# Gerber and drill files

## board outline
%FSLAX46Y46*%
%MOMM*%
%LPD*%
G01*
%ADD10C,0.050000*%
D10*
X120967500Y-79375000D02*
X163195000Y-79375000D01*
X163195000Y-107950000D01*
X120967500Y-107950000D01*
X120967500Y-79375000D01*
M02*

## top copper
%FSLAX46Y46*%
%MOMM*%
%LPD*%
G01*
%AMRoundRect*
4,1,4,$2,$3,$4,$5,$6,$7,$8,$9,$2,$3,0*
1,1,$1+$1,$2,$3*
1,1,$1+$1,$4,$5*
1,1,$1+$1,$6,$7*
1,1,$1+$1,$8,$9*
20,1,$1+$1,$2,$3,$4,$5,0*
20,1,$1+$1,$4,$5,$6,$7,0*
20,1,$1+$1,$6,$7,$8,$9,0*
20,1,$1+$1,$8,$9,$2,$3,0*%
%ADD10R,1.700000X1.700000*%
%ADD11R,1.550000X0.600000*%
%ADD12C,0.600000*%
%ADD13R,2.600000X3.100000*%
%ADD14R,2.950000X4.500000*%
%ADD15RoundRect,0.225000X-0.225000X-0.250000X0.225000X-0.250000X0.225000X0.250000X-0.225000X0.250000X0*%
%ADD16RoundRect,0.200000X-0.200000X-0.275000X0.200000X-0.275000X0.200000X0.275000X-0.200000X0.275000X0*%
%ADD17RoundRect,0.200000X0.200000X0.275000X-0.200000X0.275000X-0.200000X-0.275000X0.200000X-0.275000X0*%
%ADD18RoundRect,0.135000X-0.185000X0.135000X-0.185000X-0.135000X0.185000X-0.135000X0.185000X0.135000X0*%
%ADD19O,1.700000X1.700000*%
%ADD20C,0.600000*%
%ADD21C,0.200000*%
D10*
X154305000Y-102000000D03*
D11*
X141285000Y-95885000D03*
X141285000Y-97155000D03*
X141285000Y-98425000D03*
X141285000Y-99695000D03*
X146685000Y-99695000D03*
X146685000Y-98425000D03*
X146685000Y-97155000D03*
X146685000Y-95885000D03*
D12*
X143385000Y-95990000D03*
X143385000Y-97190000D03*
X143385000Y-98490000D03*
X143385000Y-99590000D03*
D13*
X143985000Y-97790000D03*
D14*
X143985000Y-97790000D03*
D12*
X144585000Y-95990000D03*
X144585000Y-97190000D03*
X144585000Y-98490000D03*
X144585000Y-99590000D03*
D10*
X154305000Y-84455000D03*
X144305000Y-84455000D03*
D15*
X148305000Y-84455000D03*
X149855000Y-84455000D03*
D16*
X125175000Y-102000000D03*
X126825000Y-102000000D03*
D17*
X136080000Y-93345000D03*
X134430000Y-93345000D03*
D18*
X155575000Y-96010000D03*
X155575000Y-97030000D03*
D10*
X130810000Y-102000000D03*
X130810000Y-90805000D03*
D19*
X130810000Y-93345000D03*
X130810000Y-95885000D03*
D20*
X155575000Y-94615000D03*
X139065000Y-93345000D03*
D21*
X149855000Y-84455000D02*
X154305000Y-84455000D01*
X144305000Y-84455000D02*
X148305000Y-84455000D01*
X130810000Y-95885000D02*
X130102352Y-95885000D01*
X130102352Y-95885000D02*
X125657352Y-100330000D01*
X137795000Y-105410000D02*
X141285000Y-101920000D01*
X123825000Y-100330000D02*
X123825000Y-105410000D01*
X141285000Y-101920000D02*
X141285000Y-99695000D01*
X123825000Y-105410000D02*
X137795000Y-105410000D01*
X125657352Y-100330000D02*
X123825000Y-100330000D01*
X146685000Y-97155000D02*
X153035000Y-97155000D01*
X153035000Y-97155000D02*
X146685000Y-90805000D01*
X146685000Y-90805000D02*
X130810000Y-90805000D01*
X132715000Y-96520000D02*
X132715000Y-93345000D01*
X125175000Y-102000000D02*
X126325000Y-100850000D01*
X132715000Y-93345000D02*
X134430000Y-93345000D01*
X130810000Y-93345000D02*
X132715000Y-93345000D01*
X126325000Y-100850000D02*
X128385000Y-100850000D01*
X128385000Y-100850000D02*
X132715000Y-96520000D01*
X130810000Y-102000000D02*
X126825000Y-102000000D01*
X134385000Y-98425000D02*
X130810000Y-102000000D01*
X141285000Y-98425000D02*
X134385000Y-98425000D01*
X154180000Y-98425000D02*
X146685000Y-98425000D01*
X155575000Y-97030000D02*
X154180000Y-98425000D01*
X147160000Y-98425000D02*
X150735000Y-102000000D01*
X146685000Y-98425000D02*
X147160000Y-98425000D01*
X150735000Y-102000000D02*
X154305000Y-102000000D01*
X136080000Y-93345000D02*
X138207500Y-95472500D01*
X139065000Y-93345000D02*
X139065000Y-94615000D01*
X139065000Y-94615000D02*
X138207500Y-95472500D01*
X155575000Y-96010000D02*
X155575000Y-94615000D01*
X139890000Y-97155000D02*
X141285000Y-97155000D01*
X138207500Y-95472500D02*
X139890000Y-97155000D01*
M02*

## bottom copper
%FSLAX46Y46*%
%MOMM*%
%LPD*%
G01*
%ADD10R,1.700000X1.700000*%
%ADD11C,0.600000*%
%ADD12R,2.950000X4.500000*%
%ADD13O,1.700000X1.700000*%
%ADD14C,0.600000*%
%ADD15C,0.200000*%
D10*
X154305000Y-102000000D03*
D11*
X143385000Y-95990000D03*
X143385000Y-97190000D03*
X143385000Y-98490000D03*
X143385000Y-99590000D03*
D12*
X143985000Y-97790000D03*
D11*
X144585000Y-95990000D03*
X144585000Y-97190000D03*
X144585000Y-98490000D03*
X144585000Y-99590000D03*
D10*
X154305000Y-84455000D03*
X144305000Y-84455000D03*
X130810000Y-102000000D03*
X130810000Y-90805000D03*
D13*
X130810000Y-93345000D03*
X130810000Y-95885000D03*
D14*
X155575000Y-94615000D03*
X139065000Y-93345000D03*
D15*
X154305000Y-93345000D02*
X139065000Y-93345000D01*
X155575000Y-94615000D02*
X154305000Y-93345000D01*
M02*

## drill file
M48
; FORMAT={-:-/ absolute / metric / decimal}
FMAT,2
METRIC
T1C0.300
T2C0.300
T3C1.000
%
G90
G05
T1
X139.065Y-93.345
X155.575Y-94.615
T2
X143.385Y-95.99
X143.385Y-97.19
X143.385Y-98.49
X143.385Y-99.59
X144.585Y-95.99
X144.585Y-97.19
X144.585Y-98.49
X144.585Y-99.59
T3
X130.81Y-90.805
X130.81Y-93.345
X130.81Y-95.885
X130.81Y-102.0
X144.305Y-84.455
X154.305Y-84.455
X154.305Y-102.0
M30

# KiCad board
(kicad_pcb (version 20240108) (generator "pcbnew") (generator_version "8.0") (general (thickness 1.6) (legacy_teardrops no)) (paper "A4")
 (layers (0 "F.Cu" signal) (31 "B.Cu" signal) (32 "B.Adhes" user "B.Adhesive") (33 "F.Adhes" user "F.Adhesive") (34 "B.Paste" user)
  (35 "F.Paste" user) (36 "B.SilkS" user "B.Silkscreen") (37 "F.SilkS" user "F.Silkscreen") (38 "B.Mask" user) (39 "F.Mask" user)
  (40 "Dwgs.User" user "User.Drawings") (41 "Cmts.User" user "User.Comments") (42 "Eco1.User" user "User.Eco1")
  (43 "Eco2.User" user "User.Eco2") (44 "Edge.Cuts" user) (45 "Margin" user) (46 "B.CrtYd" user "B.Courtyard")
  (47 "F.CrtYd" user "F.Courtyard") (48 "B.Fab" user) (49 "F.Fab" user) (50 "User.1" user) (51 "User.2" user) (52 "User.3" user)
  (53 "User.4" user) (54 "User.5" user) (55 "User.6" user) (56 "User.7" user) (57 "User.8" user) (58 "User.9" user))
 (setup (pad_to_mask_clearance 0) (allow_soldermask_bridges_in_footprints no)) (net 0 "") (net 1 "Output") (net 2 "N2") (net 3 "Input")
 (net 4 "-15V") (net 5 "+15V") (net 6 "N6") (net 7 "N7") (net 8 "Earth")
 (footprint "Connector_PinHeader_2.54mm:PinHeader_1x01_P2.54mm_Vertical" (layer "F.Cu") (at 154.305 102)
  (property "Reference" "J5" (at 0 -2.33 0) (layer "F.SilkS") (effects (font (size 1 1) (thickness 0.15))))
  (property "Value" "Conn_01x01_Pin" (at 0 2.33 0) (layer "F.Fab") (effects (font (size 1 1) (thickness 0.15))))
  (pad "1" thru_hole rect (at 0 0) (size 1.7 1.7) (drill 1) (layers "*.Cu" "*.Mask") (remove_unused_layers no) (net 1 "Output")))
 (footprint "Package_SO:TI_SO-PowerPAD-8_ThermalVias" (layer "F.Cu") (at 143.985 97.79)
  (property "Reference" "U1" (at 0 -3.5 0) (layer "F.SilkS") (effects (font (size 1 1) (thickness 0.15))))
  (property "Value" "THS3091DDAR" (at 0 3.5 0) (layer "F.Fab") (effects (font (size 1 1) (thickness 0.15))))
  (pad "1" smd rect (at -2.7 -1.905) (size 1.55 0.6) (layers "F.Cu" "F.Paste" "F.Mask"))
  (pad "2" smd rect (at -2.7 -0.635) (size 1.55 0.6) (layers "F.Cu" "F.Paste" "F.Mask") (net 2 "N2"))
  (pad "3" smd rect (at -2.7 0.635) (size 1.55 0.6) (layers "F.Cu" "F.Paste" "F.Mask") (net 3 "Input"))
  (pad "4" smd rect (at -2.7 1.905) (size 1.55 0.6) (layers "F.Cu" "F.Paste" "F.Mask") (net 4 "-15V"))
  (pad "5" smd rect (at 2.7 1.905) (size 1.55 0.6) (layers "F.Cu" "F.Paste" "F.Mask"))
  (pad "6" smd rect (at 2.7 0.635) (size 1.55 0.6) (layers "F.Cu" "F.Paste" "F.Mask") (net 1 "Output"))
  (pad "7" smd rect (at 2.7 -0.635) (size 1.55 0.6) (layers "F.Cu" "F.Paste" "F.Mask") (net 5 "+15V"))
  (pad "8" smd rect (at 2.7 -1.905) (size 1.55 0.6) (layers "F.Cu" "F.Paste" "F.Mask"))
  (pad "9" thru_hole circle (at -0.6 -1.8) (size 0.6 0.6) (drill 0.3) (layers "*.Cu") (remove_unused_layers no))
  (pad "9" thru_hole circle (at -0.6 -0.6) (size 0.6 0.6) (drill 0.3) (layers "*.Cu") (remove_unused_layers no))
  (pad "9" thru_hole circle (at -0.6 0.7) (size 0.6 0.6) (drill 0.3) (layers "*.Cu") (remove_unused_layers no))
  (pad "9" thru_hole circle (at -0.6 1.8) (size 0.6 0.6) (drill 0.3) (layers "*.Cu") (remove_unused_layers no))
  (pad "9" smd rect (at 0 0) (size 2.6 3.1) (layers "F.Cu" "F.Paste" "F.Mask")) (pad "9" smd rect (at 0 0) (size 2.95 4.5) (layers "F.Cu"))
  (pad "9" smd rect (at 0 0) (size 2.95 4.5) (layers "B.Cu"))
  (pad "9" thru_hole circle (at 0.6 -1.8) (size 0.6 0.6) (drill 0.3) (layers "*.Cu") (remove_unused_layers no))
  (pad "9" thru_hole circle (at 0.6 -0.6) (size 0.6 0.6) (drill 0.3) (layers "*.Cu") (remove_unused_layers no))
  (pad "9" thru_hole circle (at 0.6 0.7) (size 0.6 0.6) (drill 0.3) (layers "*.Cu") (remove_unused_layers no))
  (pad "9" thru_hole circle (at 0.6 1.8) (size 0.6 0.6) (drill 0.3) (layers "*.Cu") (remove_unused_layers no)))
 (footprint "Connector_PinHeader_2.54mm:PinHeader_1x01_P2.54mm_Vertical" (layer "F.Cu") (at 154.305 84.455)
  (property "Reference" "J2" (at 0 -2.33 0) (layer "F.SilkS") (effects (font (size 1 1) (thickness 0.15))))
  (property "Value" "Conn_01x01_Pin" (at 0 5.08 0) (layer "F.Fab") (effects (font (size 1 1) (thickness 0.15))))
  (pad "1" thru_hole rect (at 0 0) (size 1.7 1.7) (drill 1) (layers "*.Cu" "*.Mask") (remove_unused_layers no) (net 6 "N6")))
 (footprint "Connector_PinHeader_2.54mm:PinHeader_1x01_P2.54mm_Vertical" (layer "F.Cu") (at 144.305 84.455)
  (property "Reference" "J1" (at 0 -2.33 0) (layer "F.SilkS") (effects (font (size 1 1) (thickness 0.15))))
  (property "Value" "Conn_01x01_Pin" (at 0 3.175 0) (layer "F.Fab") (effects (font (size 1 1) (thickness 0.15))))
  (pad "1" thru_hole rect (at 0 0) (size 1.7 1.7) (drill 1) (layers "*.Cu" "*.Mask") (remove_unused_layers no) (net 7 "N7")))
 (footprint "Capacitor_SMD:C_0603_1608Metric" (layer "F.Cu") (at 149.08 84.455)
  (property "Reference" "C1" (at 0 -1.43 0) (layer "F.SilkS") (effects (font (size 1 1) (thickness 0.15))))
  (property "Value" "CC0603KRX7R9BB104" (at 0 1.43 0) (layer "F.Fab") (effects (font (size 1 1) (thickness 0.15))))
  (pad "1" smd roundrect (at -0.775 0) (size 0.9 0.95) (layers "F.Cu" "F.Paste" "F.Mask") (roundrect_rratio 0.25) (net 7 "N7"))
  (pad "2" smd roundrect (at 0.775 0) (size 0.9 0.95) (layers "F.Cu" "F.Paste" "F.Mask") (roundrect_rratio 0.25) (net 6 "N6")))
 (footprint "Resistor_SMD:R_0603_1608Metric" (layer "F.Cu") (at 126 102)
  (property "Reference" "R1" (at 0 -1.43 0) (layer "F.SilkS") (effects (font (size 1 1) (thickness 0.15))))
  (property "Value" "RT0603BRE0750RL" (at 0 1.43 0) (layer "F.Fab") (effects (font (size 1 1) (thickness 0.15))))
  (pad "1" smd roundrect (at -0.825 0) (size 0.8 0.95) (layers "F.Cu" "F.Paste" "F.Mask") (roundrect_rratio 0.25) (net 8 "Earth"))
  (pad "2" smd roundrect (at 0.825 0) (size 0.8 0.95) (layers "F.Cu" "F.Paste" "F.Mask") (roundrect_rratio 0.25) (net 3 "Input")))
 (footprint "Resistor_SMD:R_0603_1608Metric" (layer "F.Cu") (at 135.255 93.345 180)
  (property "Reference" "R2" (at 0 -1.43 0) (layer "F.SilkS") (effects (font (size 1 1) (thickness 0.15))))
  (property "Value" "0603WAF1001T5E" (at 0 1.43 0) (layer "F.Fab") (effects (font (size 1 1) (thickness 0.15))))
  (pad "1" smd roundrect (at -0.825 0 180) (size 0.8 0.95) (layers "F.Cu" "F.Paste" "F.Mask") (roundrect_rratio 0.25) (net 2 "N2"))
  (pad "2" smd roundrect (at 0.825 0 180) (size 0.8 0.95) (layers "F.Cu" "F.Paste" "F.Mask") (roundrect_rratio 0.25) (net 8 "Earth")))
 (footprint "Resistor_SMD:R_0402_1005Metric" (layer "F.Cu") (at 155.575 96.52 -90)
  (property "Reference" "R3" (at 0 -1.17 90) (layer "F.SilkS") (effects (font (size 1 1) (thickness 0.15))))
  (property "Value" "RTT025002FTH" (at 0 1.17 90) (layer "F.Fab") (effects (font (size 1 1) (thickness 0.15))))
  (pad "1" smd roundrect (at -0.51 0 270) (size 0.54 0.64) (layers "F.Cu" "F.Paste" "F.Mask") (roundrect_rratio 0.25) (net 2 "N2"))
  (pad "2" smd roundrect (at 0.51 0 270) (size 0.54 0.64) (layers "F.Cu" "F.Paste" "F.Mask") (roundrect_rratio 0.25) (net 1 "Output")))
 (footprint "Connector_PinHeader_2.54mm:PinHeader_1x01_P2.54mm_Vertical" (layer "F.Cu") (at 130.81 102)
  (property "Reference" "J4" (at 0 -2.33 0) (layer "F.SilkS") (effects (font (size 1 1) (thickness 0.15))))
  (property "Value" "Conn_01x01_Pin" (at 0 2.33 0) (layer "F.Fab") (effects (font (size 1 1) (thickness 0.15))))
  (pad "1" thru_hole rect (at 0 0) (size 1.7 1.7) (drill 1) (layers "*.Cu" "*.Mask") (remove_unused_layers no) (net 3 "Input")))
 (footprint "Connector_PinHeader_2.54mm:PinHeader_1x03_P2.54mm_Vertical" (layer "F.Cu") (at 130.81 90.805)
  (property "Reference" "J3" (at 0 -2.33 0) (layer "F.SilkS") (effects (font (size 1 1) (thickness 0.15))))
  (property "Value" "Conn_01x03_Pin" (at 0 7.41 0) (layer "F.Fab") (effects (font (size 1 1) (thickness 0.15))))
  (pad "1" thru_hole rect (at 0 0) (size 1.7 1.7) (drill 1) (layers "*.Cu" "*.Mask") (remove_unused_layers no) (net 5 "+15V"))
  (pad "2" thru_hole oval (at 0 2.54) (size 1.7 1.7) (drill 1) (layers "*.Cu" "*.Mask") (remove_unused_layers no) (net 8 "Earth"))
  (pad "3" thru_hole oval (at 0 5.08) (size 1.7 1.7) (drill 1) (layers "*.Cu" "*.Mask") (remove_unused_layers no) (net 4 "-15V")))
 (gr_rect (start 120.9675 79.375) (end 163.195 107.95) (stroke (width 0.05) (type default)) (fill none) (layer "Edge.Cuts"))
 (segment (start 149.855 84.455) (end 154.305 84.455) (width 0.2) (layer "F.Cu") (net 6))
 (segment (start 144.305 84.455) (end 148.305 84.455) (width 0.2) (layer "F.Cu") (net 7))
 (segment (start 130.81 95.885) (end 130.102352 95.885) (width 0.2) (layer "F.Cu") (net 4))
 (segment (start 130.102352 95.885) (end 125.657352 100.33) (width 0.2) (layer "F.Cu") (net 4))
 (segment (start 137.795 105.41) (end 141.285 101.92) (width 0.2) (layer "F.Cu") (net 4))
 (segment (start 123.825 100.33) (end 123.825 105.41) (width 0.2) (layer "F.Cu") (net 4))
 (segment (start 141.285 101.92) (end 141.285 99.695) (width 0.2) (layer "F.Cu") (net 4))
 (segment (start 123.825 105.41) (end 137.795 105.41) (width 0.2) (layer "F.Cu") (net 4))
 (segment (start 125.657352 100.33) (end 123.825 100.33) (width 0.2) (layer "F.Cu") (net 4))
 (segment (start 146.685 97.155) (end 153.035 97.155) (width 0.2) (layer "F.Cu") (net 5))
 (segment (start 153.035 97.155) (end 146.685 90.805) (width 0.2) (layer "F.Cu") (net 5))
 (segment (start 146.685 90.805) (end 130.81 90.805) (width 0.2) (layer "F.Cu") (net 5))
 (segment (start 132.715 96.52) (end 132.715 93.345) (width 0.2) (layer "F.Cu") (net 8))
 (segment (start 125.175 102) (end 126.325 100.85) (width 0.2) (layer "F.Cu") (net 8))
 (segment (start 132.715 93.345) (end 134.43 93.345) (width 0.2) (layer "F.Cu") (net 8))
 (segment (start 130.81 93.345) (end 132.715 93.345) (width 0.2) (layer "F.Cu") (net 8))
 (segment (start 126.325 100.85) (end 128.385 100.85) (width 0.2) (layer "F.Cu") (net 8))
 (segment (start 128.385 100.85) (end 132.715 96.52) (width 0.2) (layer "F.Cu") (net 8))
 (segment (start 130.81 102) (end 126.825 102) (width 0.2) (layer "F.Cu") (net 3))
 (segment (start 134.385 98.425) (end 130.81 102) (width 0.2) (layer "F.Cu") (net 3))
 (segment (start 141.285 98.425) (end 134.385 98.425) (width 0.2) (layer "F.Cu") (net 3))
 (segment (start 154.18 98.425) (end 146.685 98.425) (width 0.2) (layer "F.Cu") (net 1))
 (segment (start 155.575 97.03) (end 154.18 98.425) (width 0.2) (layer "F.Cu") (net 1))
 (segment (start 147.16 98.425) (end 150.735 102) (width 0.2) (layer "F.Cu") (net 1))
 (segment (start 146.685 98.425) (end 147.16 98.425) (width 0.2) (layer "F.Cu") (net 1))
 (segment (start 150.735 102) (end 154.305 102) (width 0.2) (layer "F.Cu") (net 1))
 (segment (start 136.08 93.345) (end 138.2075 95.4725) (width 0.2) (layer "F.Cu") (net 2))
 (segment (start 139.065 93.345) (end 139.065 94.615) (width 0.2) (layer "F.Cu") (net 2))
 (segment (start 139.065 94.615) (end 138.2075 95.4725) (width 0.2) (layer "F.Cu") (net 2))
 (segment (start 155.575 96.01) (end 155.575 94.615) (width 0.2) (layer "F.Cu") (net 2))
 (segment (start 139.89 97.155) (end 141.285 97.155) (width 0.2) (layer "F.Cu") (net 2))
 (segment (start 138.2075 95.4725) (end 139.89 97.155) (width 0.2) (layer "F.Cu") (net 2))
 (via (at 155.575 94.615) (size 0.6) (drill 0.3) (layers "F.Cu" "B.Cu") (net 2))
 (via (at 139.065 93.345) (size 0.6) (drill 0.3) (layers "F.Cu" "B.Cu") (free yes) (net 2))
 (segment (start 154.305 93.345) (end 139.065 93.345) (width 0.2) (layer "B.Cu") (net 2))
 (segment (start 155.575 94.615) (end 154.305 93.345) (width 0.2) (layer "B.Cu") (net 2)))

